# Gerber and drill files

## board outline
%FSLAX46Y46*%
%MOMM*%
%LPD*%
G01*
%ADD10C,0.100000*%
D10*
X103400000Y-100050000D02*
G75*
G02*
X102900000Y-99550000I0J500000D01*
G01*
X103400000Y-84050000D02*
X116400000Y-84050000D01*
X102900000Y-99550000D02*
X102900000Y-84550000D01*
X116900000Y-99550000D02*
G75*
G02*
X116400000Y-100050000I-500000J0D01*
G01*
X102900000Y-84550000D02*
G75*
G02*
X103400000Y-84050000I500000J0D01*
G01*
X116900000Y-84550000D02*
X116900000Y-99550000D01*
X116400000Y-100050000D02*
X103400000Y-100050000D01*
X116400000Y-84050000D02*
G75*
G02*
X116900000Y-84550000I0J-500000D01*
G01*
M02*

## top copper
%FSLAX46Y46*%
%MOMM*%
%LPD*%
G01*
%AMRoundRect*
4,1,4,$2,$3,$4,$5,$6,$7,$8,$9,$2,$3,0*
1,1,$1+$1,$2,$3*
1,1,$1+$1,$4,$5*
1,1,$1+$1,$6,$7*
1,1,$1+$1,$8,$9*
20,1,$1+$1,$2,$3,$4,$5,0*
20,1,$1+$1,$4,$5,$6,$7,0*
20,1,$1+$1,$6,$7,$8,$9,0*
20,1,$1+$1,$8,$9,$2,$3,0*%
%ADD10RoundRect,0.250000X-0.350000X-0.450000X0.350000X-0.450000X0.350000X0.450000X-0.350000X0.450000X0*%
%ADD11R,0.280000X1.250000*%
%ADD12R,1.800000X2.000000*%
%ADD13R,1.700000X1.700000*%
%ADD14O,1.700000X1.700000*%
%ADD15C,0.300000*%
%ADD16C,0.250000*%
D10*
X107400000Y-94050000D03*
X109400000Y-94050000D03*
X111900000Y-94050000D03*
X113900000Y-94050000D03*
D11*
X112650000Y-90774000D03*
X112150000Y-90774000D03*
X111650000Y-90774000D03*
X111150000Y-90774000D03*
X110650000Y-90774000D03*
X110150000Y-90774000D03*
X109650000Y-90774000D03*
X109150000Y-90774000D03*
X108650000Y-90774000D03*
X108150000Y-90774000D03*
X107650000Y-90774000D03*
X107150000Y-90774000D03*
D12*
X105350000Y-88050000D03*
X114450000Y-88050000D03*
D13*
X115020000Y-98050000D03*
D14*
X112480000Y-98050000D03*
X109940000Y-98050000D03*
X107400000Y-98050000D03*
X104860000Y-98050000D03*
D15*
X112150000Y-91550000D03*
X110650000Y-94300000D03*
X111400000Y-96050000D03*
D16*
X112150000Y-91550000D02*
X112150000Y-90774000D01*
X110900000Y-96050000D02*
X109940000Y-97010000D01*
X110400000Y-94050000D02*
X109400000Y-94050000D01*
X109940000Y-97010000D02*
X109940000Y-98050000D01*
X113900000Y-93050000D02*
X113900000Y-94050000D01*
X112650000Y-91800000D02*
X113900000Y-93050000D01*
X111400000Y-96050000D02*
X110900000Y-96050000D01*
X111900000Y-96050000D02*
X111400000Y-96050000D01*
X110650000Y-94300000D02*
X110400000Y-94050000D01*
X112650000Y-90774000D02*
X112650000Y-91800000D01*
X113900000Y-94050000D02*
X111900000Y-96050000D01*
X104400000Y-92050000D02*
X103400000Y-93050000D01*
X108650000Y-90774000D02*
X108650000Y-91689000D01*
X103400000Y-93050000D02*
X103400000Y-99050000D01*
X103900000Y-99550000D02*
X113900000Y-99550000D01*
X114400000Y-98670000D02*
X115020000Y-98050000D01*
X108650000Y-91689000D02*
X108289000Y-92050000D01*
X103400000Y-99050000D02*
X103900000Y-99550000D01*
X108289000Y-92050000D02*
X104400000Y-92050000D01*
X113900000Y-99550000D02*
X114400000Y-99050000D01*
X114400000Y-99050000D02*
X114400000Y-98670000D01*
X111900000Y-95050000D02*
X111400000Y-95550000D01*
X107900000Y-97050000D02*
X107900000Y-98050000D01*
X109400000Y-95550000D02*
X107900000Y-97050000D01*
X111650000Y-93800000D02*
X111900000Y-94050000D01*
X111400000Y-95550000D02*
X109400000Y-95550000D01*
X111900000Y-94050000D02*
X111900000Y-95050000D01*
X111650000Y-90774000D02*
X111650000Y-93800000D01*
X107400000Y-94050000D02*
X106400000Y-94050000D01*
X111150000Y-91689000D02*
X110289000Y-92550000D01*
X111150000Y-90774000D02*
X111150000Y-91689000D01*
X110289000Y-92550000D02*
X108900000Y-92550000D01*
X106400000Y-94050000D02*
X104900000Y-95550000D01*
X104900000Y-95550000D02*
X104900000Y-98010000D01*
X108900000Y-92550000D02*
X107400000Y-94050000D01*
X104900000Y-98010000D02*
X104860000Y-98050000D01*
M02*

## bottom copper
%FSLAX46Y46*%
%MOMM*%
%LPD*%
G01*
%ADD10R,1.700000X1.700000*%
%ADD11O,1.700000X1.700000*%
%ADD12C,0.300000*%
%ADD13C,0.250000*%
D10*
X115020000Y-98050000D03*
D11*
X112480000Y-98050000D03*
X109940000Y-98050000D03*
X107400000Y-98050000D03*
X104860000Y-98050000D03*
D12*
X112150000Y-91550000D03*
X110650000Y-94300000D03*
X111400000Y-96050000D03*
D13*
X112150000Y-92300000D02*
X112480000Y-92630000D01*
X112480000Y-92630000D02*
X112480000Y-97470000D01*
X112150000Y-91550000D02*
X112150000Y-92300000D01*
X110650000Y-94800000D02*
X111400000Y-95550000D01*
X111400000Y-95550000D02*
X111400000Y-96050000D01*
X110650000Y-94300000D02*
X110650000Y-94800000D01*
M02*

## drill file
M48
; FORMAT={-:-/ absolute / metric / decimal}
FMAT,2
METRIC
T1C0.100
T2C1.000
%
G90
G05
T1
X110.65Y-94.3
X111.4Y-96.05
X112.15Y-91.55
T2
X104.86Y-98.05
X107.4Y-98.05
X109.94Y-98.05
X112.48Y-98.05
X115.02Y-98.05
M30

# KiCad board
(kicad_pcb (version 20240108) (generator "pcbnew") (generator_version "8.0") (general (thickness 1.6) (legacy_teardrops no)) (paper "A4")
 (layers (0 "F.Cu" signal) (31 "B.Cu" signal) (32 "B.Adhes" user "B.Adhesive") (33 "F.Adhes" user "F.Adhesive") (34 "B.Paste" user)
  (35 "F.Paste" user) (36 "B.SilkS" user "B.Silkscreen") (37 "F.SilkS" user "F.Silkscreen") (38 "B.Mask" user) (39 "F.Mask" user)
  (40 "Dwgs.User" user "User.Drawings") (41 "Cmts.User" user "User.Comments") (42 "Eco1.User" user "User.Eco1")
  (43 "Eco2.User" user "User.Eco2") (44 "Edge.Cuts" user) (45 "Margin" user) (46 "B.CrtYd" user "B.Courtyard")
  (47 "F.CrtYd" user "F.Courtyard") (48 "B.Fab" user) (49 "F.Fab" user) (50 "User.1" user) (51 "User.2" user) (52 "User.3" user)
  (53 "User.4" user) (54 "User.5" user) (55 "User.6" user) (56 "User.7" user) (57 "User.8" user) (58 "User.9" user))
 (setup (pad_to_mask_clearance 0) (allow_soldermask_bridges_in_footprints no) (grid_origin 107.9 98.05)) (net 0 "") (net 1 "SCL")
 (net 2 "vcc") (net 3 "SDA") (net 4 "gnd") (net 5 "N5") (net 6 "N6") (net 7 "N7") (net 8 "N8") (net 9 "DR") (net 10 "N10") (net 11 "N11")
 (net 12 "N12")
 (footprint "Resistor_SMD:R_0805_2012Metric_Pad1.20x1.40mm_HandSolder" (layer "F.Cu") (at 108.4 94.05)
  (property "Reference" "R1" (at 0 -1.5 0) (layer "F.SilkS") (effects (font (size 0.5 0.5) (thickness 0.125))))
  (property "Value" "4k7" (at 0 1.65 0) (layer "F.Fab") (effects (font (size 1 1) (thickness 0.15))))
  (pad "1" smd roundrect (at -1 0) (size 1.2 1.4) (layers "F.Cu" "F.Paste" "F.Mask") (roundrect_rratio 0.208333) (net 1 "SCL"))
  (pad "2" smd roundrect (at 1 0) (size 1.2 1.4) (layers "F.Cu" "F.Paste" "F.Mask") (roundrect_rratio 0.208333) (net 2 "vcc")))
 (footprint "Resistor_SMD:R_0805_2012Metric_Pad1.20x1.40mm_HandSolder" (layer "F.Cu") (at 112.9 94.05)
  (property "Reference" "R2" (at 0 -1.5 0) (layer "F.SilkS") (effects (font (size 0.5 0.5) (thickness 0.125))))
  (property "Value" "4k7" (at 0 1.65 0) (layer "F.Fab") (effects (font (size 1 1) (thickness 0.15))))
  (pad "1" smd roundrect (at -1 0) (size 1.2 1.4) (layers "F.Cu" "F.Paste" "F.Mask") (roundrect_rratio 0.208333) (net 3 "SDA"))
  (pad "2" smd roundrect (at 1 0) (size 1.2 1.4) (layers "F.Cu" "F.Paste" "F.Mask") (roundrect_rratio 0.208333) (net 2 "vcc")))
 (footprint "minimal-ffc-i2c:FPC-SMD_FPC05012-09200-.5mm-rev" (layer "F.Cu") (at 109.9 89.412 180)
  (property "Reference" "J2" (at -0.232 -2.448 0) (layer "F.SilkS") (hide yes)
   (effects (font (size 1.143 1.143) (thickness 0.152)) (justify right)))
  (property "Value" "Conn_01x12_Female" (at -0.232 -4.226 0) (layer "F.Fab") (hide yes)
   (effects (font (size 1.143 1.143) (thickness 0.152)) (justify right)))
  (pad "1" smd rect (at -2.75 -1.362 180) (size 0.28 1.25) (layers "F.Cu" "F.Paste" "F.Mask") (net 2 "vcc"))
  (pad "2" smd rect (at -2.25 -1.362 180) (size 0.28 1.25) (layers "F.Cu" "F.Paste" "F.Mask") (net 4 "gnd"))
  (pad "3" smd rect (at -1.75 -1.362 180) (size 0.28 1.25) (layers "F.Cu" "F.Paste" "F.Mask") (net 3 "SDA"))
  (pad "4" smd rect (at -1.25 -1.362 180) (size 0.28 1.25) (layers "F.Cu" "F.Paste" "F.Mask") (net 1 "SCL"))
  (pad "5" smd rect (at -0.75 -1.362 180) (size 0.28 1.25) (layers "F.Cu" "F.Paste" "F.Mask") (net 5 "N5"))
  (pad "6" smd rect (at -0.25 -1.362 180) (size 0.28 1.25) (layers "F.Cu" "F.Paste" "F.Mask") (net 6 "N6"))
  (pad "7" smd rect (at 0.25 -1.362 180) (size 0.28 1.25) (layers "F.Cu" "F.Paste" "F.Mask") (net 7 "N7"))
  (pad "8" smd rect (at 0.75 -1.362 180) (size 0.28 1.25) (layers "F.Cu" "F.Paste" "F.Mask") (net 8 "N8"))
  (pad "9" smd rect (at 1.25 -1.362 180) (size 0.28 1.25) (layers "F.Cu" "F.Paste" "F.Mask") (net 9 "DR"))
  (pad "10" smd rect (at 1.75 -1.362 180) (size 0.28 1.25) (layers "F.Cu" "F.Paste" "F.Mask") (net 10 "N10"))
  (pad "11" smd rect (at 2.25 -1.362 180) (size 0.28 1.25) (layers "F.Cu" "F.Paste" "F.Mask") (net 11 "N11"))
  (pad "12" smd rect (at 2.75 -1.362 180) (size 0.28 1.25) (layers "F.Cu" "F.Paste" "F.Mask") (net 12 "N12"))
  (pad "13" smd rect (at 4.55 1.362 180) (size 1.8 2) (layers "F.Cu" "F.Paste" "F.Mask"))
  (pad "14" smd rect (at -4.55 1.362 180) (size 1.8 2) (layers "F.Cu" "F.Paste" "F.Mask")))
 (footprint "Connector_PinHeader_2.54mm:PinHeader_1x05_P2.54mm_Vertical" (layer "B.Cu") (at 115.02 98.05 90)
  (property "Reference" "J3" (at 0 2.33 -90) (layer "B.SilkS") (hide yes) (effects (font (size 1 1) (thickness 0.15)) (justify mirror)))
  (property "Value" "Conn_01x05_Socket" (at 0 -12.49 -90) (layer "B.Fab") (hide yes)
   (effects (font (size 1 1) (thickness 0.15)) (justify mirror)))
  (pad "1" thru_hole rect (at 0 0 90) (size 1.7 1.7) (drill 1) (layers "*.Cu" "*.Mask") (remove_unused_layers no) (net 9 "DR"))
  (pad "2" thru_hole oval (at 0 -2.54 90) (size 1.7 1.7) (drill 1) (layers "*.Cu" "*.Mask") (remove_unused_layers no) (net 4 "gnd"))
  (pad "3" thru_hole oval (at 0 -5.08 90) (size 1.7 1.7) (drill 1) (layers "*.Cu" "*.Mask") (remove_unused_layers no) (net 2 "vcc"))
  (pad "4" thru_hole oval (at 0 -7.62 90) (size 1.7 1.7) (drill 1) (layers "*.Cu" "*.Mask") (remove_unused_layers no) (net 3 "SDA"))
  (pad "5" thru_hole oval (at 0 -10.16 90) (size 1.7 1.7) (drill 1) (layers "*.Cu" "*.Mask") (remove_unused_layers no) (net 1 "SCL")))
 (gr_arc (start 103.4 100.05) (mid 103.046447 99.903553) (end 102.9 99.55) (stroke (width 0.1) (type default)) (layer "Edge.Cuts"))
 (gr_line (start 103.4 84.05) (end 116.4 84.05) (stroke (width 0.1) (type default)) (layer "Edge.Cuts"))
 (gr_line (start 102.9 99.55) (end 102.9 84.55) (stroke (width 0.1) (type default)) (layer "Edge.Cuts"))
 (gr_arc (start 116.9 99.55) (mid 116.753553 99.903553) (end 116.4 100.05) (stroke (width 0.1) (type default)) (layer "Edge.Cuts"))
 (gr_arc (start 102.9 84.55) (mid 103.046447 84.196447) (end 103.4 84.05) (stroke (width 0.1) (type default)) (layer "Edge.Cuts"))
 (gr_line (start 116.9 84.55) (end 116.9 99.55) (stroke (width 0.1) (type default)) (layer "Edge.Cuts"))
 (gr_line (start 116.4 100.05) (end 103.4 100.05) (stroke (width 0.1) (type default)) (layer "Edge.Cuts"))
 (gr_arc (start 116.4 84.05) (mid 116.753553 84.196447) (end 116.9 84.55) (stroke (width 0.1) (type default)) (layer "Edge.Cuts"))
 (segment (start 112.15 91.55) (end 112.15 90.774) (width 0.25) (layer "F.Cu") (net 4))
 (via (at 112.15 91.55) (size 0.3) (drill 0.1) (layers "F.Cu" "B.Cu") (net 4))
 (segment (start 112.15 92.3) (end 112.48 92.63) (width 0.25) (layer "B.Cu") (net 4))
 (segment (start 112.48 92.63) (end 112.48 97.47) (width 0.25) (layer "B.Cu") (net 4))
 (segment (start 112.15 91.55) (end 112.15 92.3) (width 0.25) (layer "B.Cu") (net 4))
 (segment (start 110.9 96.05) (end 109.94 97.01) (width 0.25) (layer "F.Cu") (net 2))
 (segment (start 110.4 94.05) (end 109.4 94.05) (width 0.25) (layer "F.Cu") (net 2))
 (segment (start 109.94 97.01) (end 109.94 98.05) (width 0.25) (layer "F.Cu") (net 2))
 (segment (start 113.9 93.05) (end 113.9 94.05) (width 0.25) (layer "F.Cu") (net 2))
 (segment (start 112.65 91.8) (end 113.9 93.05) (width 0.25) (layer "F.Cu") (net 2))
 (segment (start 111.4 96.05) (end 110.9 96.05) (width 0.25) (layer "F.Cu") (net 2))
 (segment (start 111.9 96.05) (end 111.4 96.05) (width 0.25) (layer "F.Cu") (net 2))
 (segment (start 110.65 94.3) (end 110.4 94.05) (width 0.25) (layer "F.Cu") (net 2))
 (segment (start 112.65 90.774) (end 112.65 91.8) (width 0.25) (layer "F.Cu") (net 2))
 (segment (start 113.9 94.05) (end 111.9 96.05) (width 0.25) (layer "F.Cu") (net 2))
 (via (at 110.65 94.3) (size 0.3) (drill 0.1) (layers "F.Cu" "B.Cu") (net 2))
 (via (at 111.4 96.05) (size 0.3) (drill 0.1) (layers "F.Cu" "B.Cu") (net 2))
 (segment (start 110.65 94.8) (end 111.4 95.55) (width 0.25) (layer "B.Cu") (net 2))
 (segment (start 111.4 95.55) (end 111.4 96.05) (width 0.25) (layer "B.Cu") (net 2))
 (segment (start 110.65 94.3) (end 110.65 94.8) (width 0.25) (layer "B.Cu") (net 2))
 (segment (start 104.4 92.05) (end 103.4 93.05) (width 0.25) (layer "F.Cu") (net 9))
 (segment (start 108.65 90.774) (end 108.65 91.689) (width 0.25) (layer "F.Cu") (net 9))
 (segment (start 103.4 93.05) (end 103.4 99.05) (width 0.25) (layer "F.Cu") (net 9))
 (segment (start 103.9 99.55) (end 113.9 99.55) (width 0.25) (layer "F.Cu") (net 9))
 (segment (start 114.4 98.67) (end 115.02 98.05) (width 0.25) (layer "F.Cu") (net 9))
 (segment (start 108.65 91.689) (end 108.289 92.05) (width 0.25) (layer "F.Cu") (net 9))
 (segment (start 103.4 99.05) (end 103.9 99.55) (width 0.25) (layer "F.Cu") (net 9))
 (segment (start 108.289 92.05) (end 104.4 92.05) (width 0.25) (layer "F.Cu") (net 9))
 (segment (start 113.9 99.55) (end 114.4 99.05) (width 0.25) (layer "F.Cu") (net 9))
 (segment (start 114.4 99.05) (end 114.4 98.67) (width 0.25) (layer "F.Cu") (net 9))
 (segment (start 111.9 95.05) (end 111.4 95.55) (width 0.25) (layer "F.Cu") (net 3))
 (segment (start 107.9 97.05) (end 107.9 98.05) (width 0.25) (layer "F.Cu") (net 3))
 (segment (start 109.4 95.55) (end 107.9 97.05) (width 0.25) (layer "F.Cu") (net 3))
 (segment (start 111.65 93.8) (end 111.9 94.05) (width 0.25) (layer "F.Cu") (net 3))
 (segment (start 111.4 95.55) (end 109.4 95.55) (width 0.25) (layer "F.Cu") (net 3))
 (segment (start 111.9 94.05) (end 111.9 95.05) (width 0.25) (layer "F.Cu") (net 3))
 (segment (start 111.65 90.774) (end 111.65 93.8) (width 0.25) (layer "F.Cu") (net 3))
 (segment (start 107.4 94.05) (end 106.4 94.05) (width 0.25) (layer "F.Cu") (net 1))
 (segment (start 111.15 91.689) (end 110.289 92.55) (width 0.25) (layer "F.Cu") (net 1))
 (segment (start 111.15 90.774) (end 111.15 91.689) (width 0.25) (layer "F.Cu") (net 1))
 (segment (start 110.289 92.55) (end 108.9 92.55) (width 0.25) (layer "F.Cu") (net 1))
 (segment (start 106.4 94.05) (end 104.9 95.55) (width 0.25) (layer "F.Cu") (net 1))
 (segment (start 104.9 95.55) (end 104.9 98.01) (width 0.25) (layer "F.Cu") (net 1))
 (segment (start 108.9 92.55) (end 107.4 94.05) (width 0.25) (layer "F.Cu") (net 1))
 (segment (start 104.9 98.01) (end 104.86 98.05) (width 0.25) (layer "F.Cu") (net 1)))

